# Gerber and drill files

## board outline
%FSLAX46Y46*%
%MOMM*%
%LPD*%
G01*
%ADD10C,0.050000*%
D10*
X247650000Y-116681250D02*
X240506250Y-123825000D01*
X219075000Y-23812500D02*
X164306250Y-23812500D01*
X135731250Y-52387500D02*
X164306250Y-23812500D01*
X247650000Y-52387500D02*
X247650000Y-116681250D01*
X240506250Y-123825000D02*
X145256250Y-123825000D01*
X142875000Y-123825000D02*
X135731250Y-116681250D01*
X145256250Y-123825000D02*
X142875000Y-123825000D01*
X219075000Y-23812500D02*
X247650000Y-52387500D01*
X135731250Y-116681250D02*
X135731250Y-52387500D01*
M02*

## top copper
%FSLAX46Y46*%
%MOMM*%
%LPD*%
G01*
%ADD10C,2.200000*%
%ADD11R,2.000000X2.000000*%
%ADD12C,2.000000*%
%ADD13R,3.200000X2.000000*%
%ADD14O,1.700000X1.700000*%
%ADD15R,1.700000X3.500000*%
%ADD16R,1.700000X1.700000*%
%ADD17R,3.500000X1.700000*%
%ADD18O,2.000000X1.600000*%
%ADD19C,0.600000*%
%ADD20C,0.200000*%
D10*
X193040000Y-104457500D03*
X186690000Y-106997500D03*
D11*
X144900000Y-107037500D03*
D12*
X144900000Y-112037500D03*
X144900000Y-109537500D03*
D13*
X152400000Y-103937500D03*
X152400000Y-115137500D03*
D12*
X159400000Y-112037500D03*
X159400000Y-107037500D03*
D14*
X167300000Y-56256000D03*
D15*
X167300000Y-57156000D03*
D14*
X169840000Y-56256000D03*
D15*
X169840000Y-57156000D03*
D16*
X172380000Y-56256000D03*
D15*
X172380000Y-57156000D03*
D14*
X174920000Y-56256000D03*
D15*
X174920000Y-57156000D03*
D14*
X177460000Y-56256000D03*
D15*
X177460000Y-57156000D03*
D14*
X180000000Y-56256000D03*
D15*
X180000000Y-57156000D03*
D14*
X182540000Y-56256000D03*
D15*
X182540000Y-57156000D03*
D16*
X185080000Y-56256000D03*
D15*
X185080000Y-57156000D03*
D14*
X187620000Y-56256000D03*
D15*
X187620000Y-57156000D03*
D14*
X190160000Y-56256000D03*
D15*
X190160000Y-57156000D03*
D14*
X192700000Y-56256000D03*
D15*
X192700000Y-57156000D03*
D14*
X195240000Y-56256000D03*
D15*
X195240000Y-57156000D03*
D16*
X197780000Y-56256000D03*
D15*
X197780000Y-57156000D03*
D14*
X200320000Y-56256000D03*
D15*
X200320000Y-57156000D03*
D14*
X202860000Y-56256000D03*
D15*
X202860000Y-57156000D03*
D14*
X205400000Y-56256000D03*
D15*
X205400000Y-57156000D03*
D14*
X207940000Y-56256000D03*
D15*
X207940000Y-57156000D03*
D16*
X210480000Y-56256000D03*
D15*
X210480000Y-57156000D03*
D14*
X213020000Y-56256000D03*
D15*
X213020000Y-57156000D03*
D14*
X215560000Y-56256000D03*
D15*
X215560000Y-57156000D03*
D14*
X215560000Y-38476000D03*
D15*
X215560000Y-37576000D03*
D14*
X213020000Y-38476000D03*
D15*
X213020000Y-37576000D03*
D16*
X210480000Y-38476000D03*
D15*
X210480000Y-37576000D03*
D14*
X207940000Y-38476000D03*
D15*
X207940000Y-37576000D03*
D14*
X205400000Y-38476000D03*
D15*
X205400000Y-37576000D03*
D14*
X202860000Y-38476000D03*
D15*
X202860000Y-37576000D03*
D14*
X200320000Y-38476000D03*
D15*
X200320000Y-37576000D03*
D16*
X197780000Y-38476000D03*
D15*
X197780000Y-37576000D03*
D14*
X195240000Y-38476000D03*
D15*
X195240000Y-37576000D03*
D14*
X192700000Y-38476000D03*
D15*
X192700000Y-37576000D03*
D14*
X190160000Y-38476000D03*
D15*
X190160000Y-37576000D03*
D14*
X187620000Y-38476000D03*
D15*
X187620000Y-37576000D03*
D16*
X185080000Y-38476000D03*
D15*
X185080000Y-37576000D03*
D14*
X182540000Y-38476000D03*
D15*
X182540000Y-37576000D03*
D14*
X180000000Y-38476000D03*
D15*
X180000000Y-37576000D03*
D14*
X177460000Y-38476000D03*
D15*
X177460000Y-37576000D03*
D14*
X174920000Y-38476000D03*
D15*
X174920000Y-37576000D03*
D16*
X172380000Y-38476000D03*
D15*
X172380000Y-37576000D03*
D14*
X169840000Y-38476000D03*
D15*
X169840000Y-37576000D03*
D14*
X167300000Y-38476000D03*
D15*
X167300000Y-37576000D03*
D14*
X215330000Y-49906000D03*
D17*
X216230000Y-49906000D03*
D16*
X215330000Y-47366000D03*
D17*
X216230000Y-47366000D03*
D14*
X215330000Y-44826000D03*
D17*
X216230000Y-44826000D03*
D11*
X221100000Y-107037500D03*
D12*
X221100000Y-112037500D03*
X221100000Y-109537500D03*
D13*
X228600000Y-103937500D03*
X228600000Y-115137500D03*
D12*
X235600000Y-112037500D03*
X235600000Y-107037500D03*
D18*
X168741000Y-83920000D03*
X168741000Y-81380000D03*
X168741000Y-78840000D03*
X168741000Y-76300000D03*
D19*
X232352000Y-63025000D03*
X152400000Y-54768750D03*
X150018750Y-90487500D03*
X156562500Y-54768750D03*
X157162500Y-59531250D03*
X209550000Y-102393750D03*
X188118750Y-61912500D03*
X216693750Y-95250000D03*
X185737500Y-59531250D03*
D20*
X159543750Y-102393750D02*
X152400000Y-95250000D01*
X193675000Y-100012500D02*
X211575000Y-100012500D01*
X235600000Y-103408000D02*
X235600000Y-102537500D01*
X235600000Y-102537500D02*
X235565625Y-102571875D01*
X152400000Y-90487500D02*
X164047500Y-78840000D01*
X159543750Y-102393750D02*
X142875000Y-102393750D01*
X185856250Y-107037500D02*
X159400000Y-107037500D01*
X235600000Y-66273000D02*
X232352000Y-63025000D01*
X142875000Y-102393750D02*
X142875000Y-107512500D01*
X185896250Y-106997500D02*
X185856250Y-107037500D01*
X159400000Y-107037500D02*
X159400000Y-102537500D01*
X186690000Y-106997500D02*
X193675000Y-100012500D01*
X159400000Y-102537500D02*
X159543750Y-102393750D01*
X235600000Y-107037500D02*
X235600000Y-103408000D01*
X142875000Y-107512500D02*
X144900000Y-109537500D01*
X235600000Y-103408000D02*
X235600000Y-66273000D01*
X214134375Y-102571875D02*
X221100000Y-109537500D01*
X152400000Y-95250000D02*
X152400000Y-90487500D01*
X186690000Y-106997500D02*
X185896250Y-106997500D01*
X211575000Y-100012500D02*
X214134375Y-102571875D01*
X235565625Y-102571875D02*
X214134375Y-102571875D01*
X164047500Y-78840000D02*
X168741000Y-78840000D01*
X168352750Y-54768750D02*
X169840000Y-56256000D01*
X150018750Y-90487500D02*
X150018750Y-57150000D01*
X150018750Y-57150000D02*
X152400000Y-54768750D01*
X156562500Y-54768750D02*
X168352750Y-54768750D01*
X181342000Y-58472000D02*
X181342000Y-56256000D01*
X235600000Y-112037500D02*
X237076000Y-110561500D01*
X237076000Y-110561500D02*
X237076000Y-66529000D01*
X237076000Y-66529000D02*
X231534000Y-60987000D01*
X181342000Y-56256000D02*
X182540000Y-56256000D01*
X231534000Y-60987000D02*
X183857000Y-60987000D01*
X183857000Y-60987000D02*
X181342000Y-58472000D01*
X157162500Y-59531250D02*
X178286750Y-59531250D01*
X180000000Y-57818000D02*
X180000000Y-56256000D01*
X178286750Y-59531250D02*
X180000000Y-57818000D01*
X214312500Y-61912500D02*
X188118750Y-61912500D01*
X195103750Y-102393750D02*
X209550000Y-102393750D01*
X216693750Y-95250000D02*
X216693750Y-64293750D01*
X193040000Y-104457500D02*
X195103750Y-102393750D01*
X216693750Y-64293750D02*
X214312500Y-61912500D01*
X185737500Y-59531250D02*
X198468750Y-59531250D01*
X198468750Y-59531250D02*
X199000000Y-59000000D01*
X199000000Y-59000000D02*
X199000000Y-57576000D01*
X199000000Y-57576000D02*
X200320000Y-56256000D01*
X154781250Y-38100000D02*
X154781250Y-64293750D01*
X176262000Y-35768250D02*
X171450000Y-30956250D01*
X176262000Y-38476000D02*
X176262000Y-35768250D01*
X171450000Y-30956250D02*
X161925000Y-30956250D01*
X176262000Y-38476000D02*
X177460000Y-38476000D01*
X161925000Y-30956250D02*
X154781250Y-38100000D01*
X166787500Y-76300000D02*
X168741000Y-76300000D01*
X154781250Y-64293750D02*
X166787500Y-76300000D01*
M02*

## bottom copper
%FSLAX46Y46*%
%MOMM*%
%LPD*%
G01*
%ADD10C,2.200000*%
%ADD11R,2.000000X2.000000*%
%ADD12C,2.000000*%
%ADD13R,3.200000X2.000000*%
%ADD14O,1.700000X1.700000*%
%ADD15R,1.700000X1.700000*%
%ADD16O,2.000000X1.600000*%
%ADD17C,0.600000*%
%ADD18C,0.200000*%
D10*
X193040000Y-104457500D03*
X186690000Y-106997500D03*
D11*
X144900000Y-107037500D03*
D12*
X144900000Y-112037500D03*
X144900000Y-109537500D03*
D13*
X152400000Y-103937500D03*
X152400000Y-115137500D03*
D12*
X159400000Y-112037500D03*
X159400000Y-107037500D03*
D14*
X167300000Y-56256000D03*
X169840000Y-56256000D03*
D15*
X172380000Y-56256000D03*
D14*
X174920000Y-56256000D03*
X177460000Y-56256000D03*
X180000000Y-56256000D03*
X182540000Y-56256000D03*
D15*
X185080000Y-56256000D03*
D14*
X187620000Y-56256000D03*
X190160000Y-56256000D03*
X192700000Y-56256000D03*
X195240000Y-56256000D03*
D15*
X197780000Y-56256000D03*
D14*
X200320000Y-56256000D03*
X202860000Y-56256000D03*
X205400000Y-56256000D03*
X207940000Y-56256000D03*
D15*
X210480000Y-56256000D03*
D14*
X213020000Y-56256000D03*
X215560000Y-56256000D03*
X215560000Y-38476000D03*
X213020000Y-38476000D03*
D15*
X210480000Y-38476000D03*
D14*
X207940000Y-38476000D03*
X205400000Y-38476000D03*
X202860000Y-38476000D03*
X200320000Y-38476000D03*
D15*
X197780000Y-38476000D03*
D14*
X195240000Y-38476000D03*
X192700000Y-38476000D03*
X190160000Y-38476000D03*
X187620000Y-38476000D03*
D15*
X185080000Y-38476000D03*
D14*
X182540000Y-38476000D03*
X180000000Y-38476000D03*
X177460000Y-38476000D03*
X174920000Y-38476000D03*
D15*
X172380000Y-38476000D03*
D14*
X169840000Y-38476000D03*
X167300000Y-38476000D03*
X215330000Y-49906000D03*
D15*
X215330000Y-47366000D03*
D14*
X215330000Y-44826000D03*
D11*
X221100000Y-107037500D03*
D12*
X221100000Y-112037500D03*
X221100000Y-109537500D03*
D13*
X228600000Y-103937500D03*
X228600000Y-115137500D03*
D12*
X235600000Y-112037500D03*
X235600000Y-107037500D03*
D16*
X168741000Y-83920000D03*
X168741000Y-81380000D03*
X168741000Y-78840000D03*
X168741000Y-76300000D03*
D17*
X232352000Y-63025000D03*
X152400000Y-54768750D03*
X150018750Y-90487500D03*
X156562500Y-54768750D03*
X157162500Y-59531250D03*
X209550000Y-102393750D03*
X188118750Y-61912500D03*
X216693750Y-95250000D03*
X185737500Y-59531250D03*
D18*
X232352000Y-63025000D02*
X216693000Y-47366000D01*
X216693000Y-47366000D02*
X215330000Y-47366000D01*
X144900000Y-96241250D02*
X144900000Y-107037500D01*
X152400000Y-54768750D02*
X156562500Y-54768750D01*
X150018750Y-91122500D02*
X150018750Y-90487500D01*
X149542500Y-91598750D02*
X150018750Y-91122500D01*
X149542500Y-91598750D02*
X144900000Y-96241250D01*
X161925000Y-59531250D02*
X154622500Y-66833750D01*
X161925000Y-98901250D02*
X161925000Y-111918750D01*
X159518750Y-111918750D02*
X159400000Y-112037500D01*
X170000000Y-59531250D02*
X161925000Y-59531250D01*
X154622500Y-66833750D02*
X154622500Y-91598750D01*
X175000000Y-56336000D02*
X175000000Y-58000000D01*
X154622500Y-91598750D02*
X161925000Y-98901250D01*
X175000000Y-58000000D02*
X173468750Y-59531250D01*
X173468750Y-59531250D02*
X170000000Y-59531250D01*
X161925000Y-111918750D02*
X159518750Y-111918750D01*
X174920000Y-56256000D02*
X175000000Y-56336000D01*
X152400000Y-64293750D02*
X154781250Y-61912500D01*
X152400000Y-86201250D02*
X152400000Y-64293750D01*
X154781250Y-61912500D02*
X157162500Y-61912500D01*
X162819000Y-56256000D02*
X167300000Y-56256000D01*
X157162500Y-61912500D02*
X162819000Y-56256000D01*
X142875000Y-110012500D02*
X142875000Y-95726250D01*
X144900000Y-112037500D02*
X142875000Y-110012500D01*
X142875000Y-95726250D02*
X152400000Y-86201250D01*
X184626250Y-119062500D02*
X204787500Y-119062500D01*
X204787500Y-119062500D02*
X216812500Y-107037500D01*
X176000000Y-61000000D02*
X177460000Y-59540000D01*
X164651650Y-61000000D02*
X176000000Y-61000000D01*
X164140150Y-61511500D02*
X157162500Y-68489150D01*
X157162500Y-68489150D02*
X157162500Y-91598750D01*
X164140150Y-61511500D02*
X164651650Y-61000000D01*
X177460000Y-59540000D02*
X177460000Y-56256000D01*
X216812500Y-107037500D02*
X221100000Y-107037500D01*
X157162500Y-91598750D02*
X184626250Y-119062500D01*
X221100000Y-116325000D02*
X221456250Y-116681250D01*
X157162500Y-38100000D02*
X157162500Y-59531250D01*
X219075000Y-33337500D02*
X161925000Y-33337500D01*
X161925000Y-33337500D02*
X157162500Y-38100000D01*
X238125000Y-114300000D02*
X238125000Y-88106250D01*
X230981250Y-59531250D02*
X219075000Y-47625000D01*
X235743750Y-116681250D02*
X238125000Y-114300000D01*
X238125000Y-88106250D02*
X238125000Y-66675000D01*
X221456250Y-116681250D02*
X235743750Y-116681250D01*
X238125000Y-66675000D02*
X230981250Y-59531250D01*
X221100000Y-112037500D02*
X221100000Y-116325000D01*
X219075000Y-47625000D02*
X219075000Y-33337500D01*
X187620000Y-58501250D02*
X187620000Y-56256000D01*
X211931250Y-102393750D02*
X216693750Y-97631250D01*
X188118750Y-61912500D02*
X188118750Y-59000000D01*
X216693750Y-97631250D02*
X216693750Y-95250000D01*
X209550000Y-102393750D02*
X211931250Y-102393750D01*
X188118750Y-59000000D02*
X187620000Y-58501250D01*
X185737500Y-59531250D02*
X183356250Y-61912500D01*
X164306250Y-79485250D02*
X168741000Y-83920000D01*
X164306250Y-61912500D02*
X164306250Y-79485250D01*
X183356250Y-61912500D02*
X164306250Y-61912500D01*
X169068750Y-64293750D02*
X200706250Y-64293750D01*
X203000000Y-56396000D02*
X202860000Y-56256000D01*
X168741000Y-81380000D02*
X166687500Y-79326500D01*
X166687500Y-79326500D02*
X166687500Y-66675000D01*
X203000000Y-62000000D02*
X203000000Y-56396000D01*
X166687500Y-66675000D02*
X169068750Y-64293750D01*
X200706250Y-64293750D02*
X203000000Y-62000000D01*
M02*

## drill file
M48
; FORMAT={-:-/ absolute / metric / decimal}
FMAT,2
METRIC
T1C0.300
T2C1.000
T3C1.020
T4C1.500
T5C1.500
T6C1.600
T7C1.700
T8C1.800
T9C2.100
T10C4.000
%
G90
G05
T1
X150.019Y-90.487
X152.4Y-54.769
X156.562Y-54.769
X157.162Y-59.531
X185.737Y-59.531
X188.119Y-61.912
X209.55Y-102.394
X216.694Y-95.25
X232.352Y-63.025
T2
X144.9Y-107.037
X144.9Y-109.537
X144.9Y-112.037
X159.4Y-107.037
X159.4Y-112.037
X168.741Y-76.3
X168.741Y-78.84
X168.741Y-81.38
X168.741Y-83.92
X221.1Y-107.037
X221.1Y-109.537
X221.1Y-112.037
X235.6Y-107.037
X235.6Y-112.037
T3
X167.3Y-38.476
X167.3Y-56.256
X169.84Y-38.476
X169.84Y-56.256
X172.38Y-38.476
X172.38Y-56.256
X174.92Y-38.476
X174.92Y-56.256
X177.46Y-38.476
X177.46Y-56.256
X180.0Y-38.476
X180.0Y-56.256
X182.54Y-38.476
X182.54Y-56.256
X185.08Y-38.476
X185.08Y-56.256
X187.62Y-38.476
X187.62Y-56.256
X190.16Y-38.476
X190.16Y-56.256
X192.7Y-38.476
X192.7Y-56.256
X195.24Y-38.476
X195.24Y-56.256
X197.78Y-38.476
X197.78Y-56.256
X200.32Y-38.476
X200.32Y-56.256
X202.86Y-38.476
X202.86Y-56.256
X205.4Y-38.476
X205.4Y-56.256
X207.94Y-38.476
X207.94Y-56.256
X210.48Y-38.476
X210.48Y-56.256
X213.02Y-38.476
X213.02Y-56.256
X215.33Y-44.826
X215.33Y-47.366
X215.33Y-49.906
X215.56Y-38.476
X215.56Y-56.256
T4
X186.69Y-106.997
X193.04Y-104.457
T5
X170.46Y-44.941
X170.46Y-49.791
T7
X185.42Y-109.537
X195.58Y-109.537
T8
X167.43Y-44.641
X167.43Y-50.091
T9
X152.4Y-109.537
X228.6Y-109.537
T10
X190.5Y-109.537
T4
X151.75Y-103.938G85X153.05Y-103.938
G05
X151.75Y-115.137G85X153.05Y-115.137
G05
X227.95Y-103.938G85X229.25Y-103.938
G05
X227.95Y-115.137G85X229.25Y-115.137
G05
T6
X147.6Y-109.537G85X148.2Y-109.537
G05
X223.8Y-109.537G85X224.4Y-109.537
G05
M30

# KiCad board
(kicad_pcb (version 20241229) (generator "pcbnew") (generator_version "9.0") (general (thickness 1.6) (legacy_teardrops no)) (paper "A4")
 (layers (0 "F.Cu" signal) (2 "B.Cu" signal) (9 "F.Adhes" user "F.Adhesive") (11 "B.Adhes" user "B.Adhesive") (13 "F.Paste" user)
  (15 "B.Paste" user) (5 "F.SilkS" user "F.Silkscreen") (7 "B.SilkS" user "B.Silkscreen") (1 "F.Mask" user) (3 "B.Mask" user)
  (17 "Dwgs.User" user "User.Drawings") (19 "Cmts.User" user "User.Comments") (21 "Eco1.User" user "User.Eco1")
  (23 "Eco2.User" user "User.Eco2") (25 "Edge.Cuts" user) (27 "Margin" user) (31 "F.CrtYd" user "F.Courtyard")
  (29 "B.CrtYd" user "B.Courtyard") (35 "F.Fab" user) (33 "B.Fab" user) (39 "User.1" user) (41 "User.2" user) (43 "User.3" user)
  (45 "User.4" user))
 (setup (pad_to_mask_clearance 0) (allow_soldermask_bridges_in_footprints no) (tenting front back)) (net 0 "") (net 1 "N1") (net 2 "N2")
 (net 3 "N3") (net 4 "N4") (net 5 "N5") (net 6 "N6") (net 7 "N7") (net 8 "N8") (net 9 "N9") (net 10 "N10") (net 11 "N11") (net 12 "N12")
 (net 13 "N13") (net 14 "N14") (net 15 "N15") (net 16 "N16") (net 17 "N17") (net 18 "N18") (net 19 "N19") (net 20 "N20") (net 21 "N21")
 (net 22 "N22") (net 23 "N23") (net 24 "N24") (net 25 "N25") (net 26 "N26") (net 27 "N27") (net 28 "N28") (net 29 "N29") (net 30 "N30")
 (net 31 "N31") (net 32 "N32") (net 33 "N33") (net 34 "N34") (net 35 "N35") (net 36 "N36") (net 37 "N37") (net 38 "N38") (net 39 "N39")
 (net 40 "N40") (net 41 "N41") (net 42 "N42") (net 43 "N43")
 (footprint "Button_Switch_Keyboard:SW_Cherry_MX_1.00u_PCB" (layer "F.Cu") (at 193.04 104.4575)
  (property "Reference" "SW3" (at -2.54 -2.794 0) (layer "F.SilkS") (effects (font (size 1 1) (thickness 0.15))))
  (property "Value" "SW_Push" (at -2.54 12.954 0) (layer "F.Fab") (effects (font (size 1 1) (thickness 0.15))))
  (pad "" np_thru_hole circle (at -7.62 5.08) (size 1.7 1.7) (drill 1.7) (layers "*.Cu" "*.Mask"))
  (pad "" np_thru_hole circle (at -2.54 5.08) (size 4 4) (drill 4) (layers "*.Cu" "*.Mask"))
  (pad "" np_thru_hole circle (at 2.54 5.08) (size 1.7 1.7) (drill 1.7) (layers "*.Cu" "*.Mask"))
  (pad "1" thru_hole circle (at 0 0) (size 2.2 2.2) (drill 1.5) (layers "*.Cu" "*.Mask") (remove_unused_layers no) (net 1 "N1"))
  (pad "2" thru_hole circle (at -6.35 2.54) (size 2.2 2.2) (drill 1.5) (layers "*.Cu" "*.Mask") (remove_unused_layers no) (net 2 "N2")))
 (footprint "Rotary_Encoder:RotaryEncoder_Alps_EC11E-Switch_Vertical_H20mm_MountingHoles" (layer "F.Cu") (at 144.9 107.0375)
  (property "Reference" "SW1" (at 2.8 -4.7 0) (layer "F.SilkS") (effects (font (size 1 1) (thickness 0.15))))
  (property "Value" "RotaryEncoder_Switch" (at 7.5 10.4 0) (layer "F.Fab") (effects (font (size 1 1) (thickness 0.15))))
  (pad "" np_thru_hole oval (at 3 2.5) (size 2.2 1.6) (drill oval 2.2 1.6) (layers "*.Mask"))
  (pad "" np_thru_hole circle (at 7.5 2.5) (size 2.1 2.1) (drill 2.1) (layers "*.Mask"))
  (pad "A" thru_hole rect (at 0 0) (size 2 2) (drill 1) (layers "*.Cu" "*.Mask") (remove_unused_layers no) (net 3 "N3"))
  (pad "B" thru_hole circle (at 0 5) (size 2 2) (drill 1) (layers "*.Cu" "*.Mask") (remove_unused_layers no) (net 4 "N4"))
  (pad "C" thru_hole circle (at 0 2.5) (size 2 2) (drill 1) (layers "*.Cu" "*.Mask") (remove_unused_layers no) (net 2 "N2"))
  (pad "MP" thru_hole rect (at 7.5 -3.1) (size 3.2 2) (drill oval 2.8 1.5) (layers "*.Cu" "*.Mask") (remove_unused_layers no))
  (pad "MP" thru_hole rect (at 7.5 8.1) (size 3.2 2) (drill oval 2.8 1.5) (layers "*.Cu" "*.Mask") (remove_unused_layers no))
  (pad "S1" thru_hole circle (at 14.5 5) (size 2 2) (drill 1) (layers "*.Cu" "*.Mask") (remove_unused_layers no) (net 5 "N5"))
  (pad "S2" thru_hole circle (at 14.5 0) (size 2 2) (drill 1) (layers "*.Cu" "*.Mask") (remove_unused_layers no) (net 2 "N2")))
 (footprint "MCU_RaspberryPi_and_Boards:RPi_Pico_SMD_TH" (layer "F.Cu") (at 191.43 47.366 90)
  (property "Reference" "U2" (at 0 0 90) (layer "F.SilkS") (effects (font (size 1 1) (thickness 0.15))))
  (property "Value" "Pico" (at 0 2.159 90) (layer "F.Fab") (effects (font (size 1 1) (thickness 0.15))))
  (pad "" np_thru_hole oval (at -2.725 -24 90) (size 1.8 1.8) (drill 1.8) (layers "*.Cu" "*.Mask"))
  (pad "" np_thru_hole oval (at -2.425 -20.97 90) (size 1.5 1.5) (drill 1.5) (layers "*.Cu" "*.Mask"))
  (pad "" np_thru_hole oval (at 2.425 -20.97 90) (size 1.5 1.5) (drill 1.5) (layers "*.Cu" "*.Mask"))
  (pad "" np_thru_hole oval (at 2.725 -24 90) (size 1.8 1.8) (drill 1.8) (layers "*.Cu" "*.Mask"))
  (pad "1" thru_hole oval (at -8.89 -24.13 90) (size 1.7 1.7) (drill 1.02) (layers "*.Cu" "*.Mask") (remove_unused_layers no) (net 4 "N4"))
  (pad "1" smd rect (at -8.89 -24.13 90) (size 3.5 1.7) (drill (offset -0.9 0)) (layers "F.Cu" "F.Mask") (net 4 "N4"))
  (pad "2" thru_hole oval (at -8.89 -21.59 90) (size 1.7 1.7) (drill 1.02) (layers "*.Cu" "*.Mask") (remove_unused_layers no) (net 3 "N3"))
  (pad "2" smd rect (at -8.89 -21.59 90) (size 3.5 1.7) (drill (offset -0.9 0)) (layers "F.Cu" "F.Mask") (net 3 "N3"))
  (pad "3" thru_hole rect (at -8.89 -19.05 90) (size 1.7 1.7) (drill 1.02) (layers "*.Cu" "*.Mask") (remove_unused_layers no) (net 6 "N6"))
  (pad "3" smd rect (at -8.89 -19.05 90) (size 3.5 1.7) (drill (offset -0.9 0)) (layers "F.Cu" "F.Mask") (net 6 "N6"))
  (pad "4" thru_hole oval (at -8.89 -16.51 90) (size 1.7 1.7) (drill 1.02) (layers "*.Cu" "*.Mask") (remove_unused_layers no) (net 5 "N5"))
  (pad "4" smd rect (at -8.89 -16.51 90) (size 3.5 1.7) (drill (offset -0.9 0)) (layers "F.Cu" "F.Mask") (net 5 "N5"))
  (pad "5" thru_hole oval (at -8.89 -13.97 90) (size 1.7 1.7) (drill 1.02) (layers "*.Cu" "*.Mask") (remove_unused_layers no) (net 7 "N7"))
  (pad "5" smd rect (at -8.89 -13.97 90) (size 3.5 1.7) (drill (offset -0.9 0)) (layers "F.Cu" "F.Mask") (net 7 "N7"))
  (pad "6" thru_hole oval (at -8.89 -11.43 90) (size 1.7 1.7) (drill 1.02) (layers "*.Cu" "*.Mask") (remove_unused_layers no) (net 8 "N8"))
  (pad "6" smd rect (at -8.89 -11.43 90) (size 3.5 1.7) (drill (offset -0.9 0)) (layers "F.Cu" "F.Mask") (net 8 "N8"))
  (pad "7" thru_hole oval (at -8.89 -8.89 90) (size 1.7 1.7) (drill 1.02) (layers "*.Cu" "*.Mask") (remove_unused_layers no) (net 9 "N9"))
  (pad "7" smd rect (at -8.89 -8.89 90) (size 3.5 1.7) (drill (offset -0.9 0)) (layers "F.Cu" "F.Mask") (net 9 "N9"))
  (pad "8" thru_hole rect (at -8.89 -6.35 90) (size 1.7 1.7) (drill 1.02) (layers "*.Cu" "*.Mask") (remove_unused_layers no) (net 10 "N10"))
  (pad "8" smd rect (at -8.89 -6.35 90) (size 3.5 1.7) (drill (offset -0.9 0)) (layers "F.Cu" "F.Mask") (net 10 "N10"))
  (pad "9" thru_hole oval (at -8.89 -3.81 90) (size 1.7 1.7) (drill 1.02) (layers "*.Cu" "*.Mask") (remove_unused_layers no) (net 1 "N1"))
  (pad "9" smd rect (at -8.89 -3.81 90) (size 3.5 1.7) (drill (offset -0.9 0)) (layers "F.Cu" "F.Mask") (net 1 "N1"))
  (pad "10" thru_hole oval (at -8.89 -1.27 90) (size 1.7 1.7) (drill 1.02) (layers "*.Cu" "*.Mask") (remove_unused_layers no) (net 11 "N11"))
  (pad "10" smd rect (at -8.89 -1.27 90) (size 3.5 1.7) (drill (offset -0.9 0)) (layers "F.Cu" "F.Mask") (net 11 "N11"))
  (pad "11" thru_hole oval (at -8.89 1.27 90) (size 1.7 1.7) (drill 1.02) (layers "*.Cu" "*.Mask") (remove_unused_layers no) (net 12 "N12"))
  (pad "11" smd rect (at -8.89 1.27 90) (size 3.5 1.7) (drill (offset -0.9 0)) (layers "F.Cu" "F.Mask") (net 12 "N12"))
  (pad "12" thru_hole oval (at -8.89 3.81 90) (size 1.7 1.7) (drill 1.02) (layers "*.Cu" "*.Mask") (remove_unused_layers no) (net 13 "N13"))
  (pad "12" smd rect (at -8.89 3.81 90) (size 3.5 1.7) (drill (offset -0.9 0)) (layers "F.Cu" "F.Mask") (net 13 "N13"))
  (pad "13" thru_hole rect (at -8.89 6.35 90) (size 1.7 1.7) (drill 1.02) (layers "*.Cu" "*.Mask") (remove_unused_layers no) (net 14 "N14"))
  (pad "13" smd rect (at -8.89 6.35 90) (size 3.5 1.7) (drill (offset -0.9 0)) (layers "F.Cu" "F.Mask") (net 14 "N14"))
  (pad "14" thru_hole oval (at -8.89 8.89 90) (size 1.7 1.7) (drill 1.02) (layers "*.Cu" "*.Mask") (remove_unused_layers no) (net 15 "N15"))
  (pad "14" smd rect (at -8.89 8.89 90) (size 3.5 1.7) (drill (offset -0.9 0)) (layers "F.Cu" "F.Mask") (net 15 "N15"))
  (pad "15" thru_hole oval (at -8.89 11.43 90) (size 1.7 1.7) (drill 1.02) (layers "*.Cu" "*.Mask") (remove_unused_layers no) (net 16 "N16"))
  (pad "15" smd rect (at -8.89 11.43 90) (size 3.5 1.7) (drill (offset -0.9 0)) (layers "F.Cu" "F.Mask") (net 16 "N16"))
  (pad "16" thru_hole oval (at -8.89 13.97 90) (size 1.7 1.7) (drill 1.02) (layers "*.Cu" "*.Mask") (remove_unused_layers no) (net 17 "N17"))
  (pad "16" smd rect (at -8.89 13.97 90) (size 3.5 1.7) (drill (offset -0.9 0)) (layers "F.Cu" "F.Mask") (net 17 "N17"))
  (pad "17" thru_hole oval (at -8.89 16.51 90) (size 1.7 1.7) (drill 1.02) (layers "*.Cu" "*.Mask") (remove_unused_layers no) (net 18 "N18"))
  (pad "17" smd rect (at -8.89 16.51 90) (size 3.5 1.7) (drill (offset -0.9 0)) (layers "F.Cu" "F.Mask") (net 18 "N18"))
  (pad "18" thru_hole rect (at -8.89 19.05 90) (size 1.7 1.7) (drill 1.02) (layers "*.Cu" "*.Mask") (remove_unused_layers no) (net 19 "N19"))
  (pad "18" smd rect (at -8.89 19.05 90) (size 3.5 1.7) (drill (offset -0.9 0)) (layers "F.Cu" "F.Mask") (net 19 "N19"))
  (pad "19" thru_hole oval (at -8.89 21.59 90) (size 1.7 1.7) (drill 1.02) (layers "*.Cu" "*.Mask") (remove_unused_layers no) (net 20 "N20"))
  (pad "19" smd rect (at -8.89 21.59 90) (size 3.5 1.7) (drill (offset -0.9 0)) (layers "F.Cu" "F.Mask") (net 20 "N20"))
  (pad "20" thru_hole oval (at -8.89 24.13 90) (size 1.7 1.7) (drill 1.02) (layers "*.Cu" "*.Mask") (remove_unused_layers no) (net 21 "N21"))
  (pad "20" smd rect (at -8.89 24.13 90) (size 3.5 1.7) (drill (offset -0.9 0)) (layers "F.Cu" "F.Mask") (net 21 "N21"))
  (pad "21" thru_hole oval (at 8.89 24.13 90) (size 1.7 1.7) (drill 1.02) (layers "*.Cu" "*.Mask") (remove_unused_layers no) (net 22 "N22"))
  (pad "21" smd rect (at 8.89 24.13 90) (size 3.5 1.7) (drill (offset 0.9 0)) (layers "F.Cu" "F.Mask") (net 22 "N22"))
  (pad "22" thru_hole oval (at 8.89 21.59 90) (size 1.7 1.7) (drill 1.02) (layers "*.Cu" "*.Mask") (remove_unused_layers no) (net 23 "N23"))
  (pad "22" smd rect (at 8.89 21.59 90) (size 3.5 1.7) (drill (offset 0.9 0)) (layers "F.Cu" "F.Mask") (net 23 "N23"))
  (pad "23" thru_hole rect (at 8.89 19.05 90) (size 1.7 1.7) (drill 1.02) (layers "*.Cu" "*.Mask") (remove_unused_layers no) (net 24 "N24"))
  (pad "23" smd rect (at 8.89 19.05 90) (size 3.5 1.7) (drill (offset 0.9 0)) (layers "F.Cu" "F.Mask") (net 24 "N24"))
  (pad "24" thru_hole oval (at 8.89 16.51 90) (size 1.7 1.7) (drill 1.02) (layers "*.Cu" "*.Mask") (remove_unused_layers no) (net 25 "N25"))
  (pad "24" smd rect (at 8.89 16.51 90) (size 3.5 1.7) (drill (offset 0.9 0)) (layers "F.Cu" "F.Mask") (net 25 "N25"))
  (pad "25" thru_hole oval (at 8.89 13.97 90) (size 1.7 1.7) (drill 1.02) (layers "*.Cu" "*.Mask") (remove_unused_layers no) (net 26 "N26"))
  (pad "25" smd rect (at 8.89 13.97 90) (size 3.5 1.7) (drill (offset 0.9 0)) (layers "F.Cu" "F.Mask") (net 26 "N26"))
  (pad "26" thru_hole oval (at 8.89 11.43 90) (size 1.7 1.7) (drill 1.02) (layers "*.Cu" "*.Mask") (remove_unused_layers no) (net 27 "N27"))
  (pad "26" smd rect (at 8.89 11.43 90) (size 3.5 1.7) (drill (offset 0.9 0)) (layers "F.Cu" "F.Mask") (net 27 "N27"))
  (pad "27" thru_hole oval (at 8.89 8.89 90) (size 1.7 1.7) (drill 1.02) (layers "*.Cu" "*.Mask") (remove_unused_layers no) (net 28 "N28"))
  (pad "27" smd rect (at 8.89 8.89 90) (size 3.5 1.7) (drill (offset 0.9 0)) (layers "F.Cu" "F.Mask") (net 28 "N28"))
  (pad "28" thru_hole rect (at 8.89 6.35 90) (size 1.7 1.7) (drill 1.02) (layers "*.Cu" "*.Mask") (remove_unused_layers no) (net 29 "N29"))
  (pad "28" smd rect (at 8.89 6.35 90) (size 3.5 1.7) (drill (offset 0.9 0)) (layers "F.Cu" "F.Mask") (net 29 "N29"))
  (pad "29" thru_hole oval (at 8.89 3.81 90) (size 1.7 1.7) (drill 1.02) (layers "*.Cu" "*.Mask") (remove_unused_layers no) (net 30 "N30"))
  (pad "29" smd rect (at 8.89 3.81 90) (size 3.5 1.7) (drill (offset 0.9 0)) (layers "F.Cu" "F.Mask") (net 30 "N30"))
  (pad "30" thru_hole oval (at 8.89 1.27 90) (size 1.7 1.7) (drill 1.02) (layers "*.Cu" "*.Mask") (remove_unused_layers no) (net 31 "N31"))
  (pad "30" smd rect (at 8.89 1.27 90) (size 3.5 1.7) (drill (offset 0.9 0)) (layers "F.Cu" "F.Mask") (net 31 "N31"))
  (pad "31" thru_hole oval (at 8.89 -1.27 90) (size 1.7 1.7) (drill 1.02) (layers "*.Cu" "*.Mask") (remove_unused_layers no) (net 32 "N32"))
  (pad "31" smd rect (at 8.89 -1.27 90) (size 3.5 1.7) (drill (offset 0.9 0)) (layers "F.Cu" "F.Mask") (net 32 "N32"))
  (pad "32" thru_hole oval (at 8.89 -3.81 90) (size 1.7 1.7) (drill 1.02) (layers "*.Cu" "*.Mask") (remove_unused_layers no) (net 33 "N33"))
  (pad "32" smd rect (at 8.89 -3.81 90) (size 3.5 1.7) (drill (offset 0.9 0)) (layers "F.Cu" "F.Mask") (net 33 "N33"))
  (pad "33" thru_hole rect (at 8.89 -6.35 90) (size 1.7 1.7) (drill 1.02) (layers "*.Cu" "*.Mask") (remove_unused_layers no) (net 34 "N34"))
  (pad "33" smd rect (at 8.89 -6.35 90) (size 3.5 1.7) (drill (offset 0.9 0)) (layers "F.Cu" "F.Mask") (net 34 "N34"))
  (pad "34" thru_hole oval (at 8.89 -8.89 90) (size 1.7 1.7) (drill 1.02) (layers "*.Cu" "*.Mask") (remove_unused_layers no) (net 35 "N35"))
  (pad "34" smd rect (at 8.89 -8.89 90) (size 3.5 1.7) (drill (offset 0.9 0)) (layers "F.Cu" "F.Mask") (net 35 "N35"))
  (pad "35" thru_hole oval (at 8.89 -11.43 90) (size 1.7 1.7) (drill 1.02) (layers "*.Cu" "*.Mask") (remove_unused_layers no) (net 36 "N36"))
  (pad "35" smd rect (at 8.89 -11.43 90) (size 3.5 1.7) (drill (offset 0.9 0)) (layers "F.Cu" "F.Mask") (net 36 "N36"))
  (pad "36" thru_hole oval (at 8.89 -13.97 90) (size 1.7 1.7) (drill 1.02) (layers "*.Cu" "*.Mask") (remove_unused_layers no) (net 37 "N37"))
  (pad "36" smd rect (at 8.89 -13.97 90) (size 3.5 1.7) (drill (offset 0.9 0)) (layers "F.Cu" "F.Mask") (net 37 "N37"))
  (pad "37" thru_hole oval (at 8.89 -16.51 90) (size 1.7 1.7) (drill 1.02) (layers "*.Cu" "*.Mask") (remove_unused_layers no) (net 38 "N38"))
  (pad "37" smd rect (at 8.89 -16.51 90) (size 3.5 1.7) (drill (offset 0.9 0)) (layers "F.Cu" "F.Mask") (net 38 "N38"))
  (pad "38" thru_hole rect (at 8.89 -19.05 90) (size 1.7 1.7) (drill 1.02) (layers "*.Cu" "*.Mask") (remove_unused_layers no) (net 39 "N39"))
  (pad "38" smd rect (at 8.89 -19.05 90) (size 3.5 1.7) (drill (offset 0.9 0)) (layers "F.Cu" "F.Mask") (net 39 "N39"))
  (pad "39" thru_hole oval (at 8.89 -21.59 90) (size 1.7 1.7) (drill 1.02) (layers "*.Cu" "*.Mask") (remove_unused_layers no) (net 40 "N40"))
  (pad "39" smd rect (at 8.89 -21.59 90) (size 3.5 1.7) (drill (offset 0.9 0)) (layers "F.Cu" "F.Mask") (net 40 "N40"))
  (pad "40" thru_hole oval (at 8.89 -24.13 90) (size 1.7 1.7) (drill 1.02) (layers "*.Cu" "*.Mask") (remove_unused_layers no) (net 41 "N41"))
  (pad "40" smd rect (at 8.89 -24.13 90) (size 3.5 1.7) (drill (offset 0.9 0)) (layers "F.Cu" "F.Mask") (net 41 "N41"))
  (pad "41" thru_hole oval (at -2.54 23.9 90) (size 1.7 1.7) (drill 1.02) (layers "*.Cu" "*.Mask") (remove_unused_layers no) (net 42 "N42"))
  (pad "41" smd rect (at -2.54 23.9 180) (size 3.5 1.7) (drill (offset -0.9 0)) (layers "F.Cu" "F.Mask") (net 42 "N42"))
  (pad "42" thru_hole rect (at 0 23.9 90) (size 1.7 1.7) (drill 1.02) (layers "*.Cu" "*.Mask") (remove_unused_layers no) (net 2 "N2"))
  (pad "42" smd rect (at 0 23.9 180) (size 3.5 1.7) (drill (offset -0.9 0)) (layers "F.Cu" "F.Mask") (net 2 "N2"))
  (pad "43" thru_hole oval (at 2.54 23.9 90) (size 1.7 1.7) (drill 1.02) (layers "*.Cu" "*.Mask") (remove_unused_layers no) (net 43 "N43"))
  (pad "43" smd rect (at 2.54 23.9 180) (size 3.5 1.7) (drill (offset -0.9 0)) (layers "F.Cu" "F.Mask") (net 43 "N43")))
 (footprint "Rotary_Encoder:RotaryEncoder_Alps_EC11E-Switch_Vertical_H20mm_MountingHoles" (layer "F.Cu") (at 221.1 107.0375)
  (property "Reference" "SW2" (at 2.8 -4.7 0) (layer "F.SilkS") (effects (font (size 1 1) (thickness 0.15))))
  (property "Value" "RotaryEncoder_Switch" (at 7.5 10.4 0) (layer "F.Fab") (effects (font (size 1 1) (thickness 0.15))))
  (pad "" np_thru_hole oval (at 3 2.5) (size 2.2 1.6) (drill oval 2.2 1.6) (layers "*.Mask"))
  (pad "" np_thru_hole circle (at 7.5 2.5) (size 2.1 2.1) (drill 2.1) (layers "*.Mask"))
  (pad "A" thru_hole rect (at 0 0) (size 2 2) (drill 1) (layers "*.Cu" "*.Mask") (remove_unused_layers no) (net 7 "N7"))
  (pad "B" thru_hole circle (at 0 5) (size 2 2) (drill 1) (layers "*.Cu" "*.Mask") (remove_unused_layers no) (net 8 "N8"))
  (pad "C" thru_hole circle (at 0 2.5) (size 2 2) (drill 1) (layers "*.Cu" "*.Mask") (remove_unused_layers no) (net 2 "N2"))
  (pad "MP" thru_hole rect (at 7.5 -3.1) (size 3.2 2) (drill oval 2.8 1.5) (layers "*.Cu" "*.Mask") (remove_unused_layers no))
  (pad "MP" thru_hole rect (at 7.5 8.1) (size 3.2 2) (drill oval 2.8 1.5) (layers "*.Cu" "*.Mask") (remove_unused_layers no))
  (pad "S1" thru_hole circle (at 14.5 5) (size 2 2) (drill 1) (layers "*.Cu" "*.Mask") (remove_unused_layers no) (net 9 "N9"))
  (pad "S2" thru_hole circle (at 14.5 0) (size 2 2) (drill 1) (layers "*.Cu" "*.Mask") (remove_unused_layers no) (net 2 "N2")))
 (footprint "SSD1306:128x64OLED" (layer "F.Cu") (at 179.341 80.3 90)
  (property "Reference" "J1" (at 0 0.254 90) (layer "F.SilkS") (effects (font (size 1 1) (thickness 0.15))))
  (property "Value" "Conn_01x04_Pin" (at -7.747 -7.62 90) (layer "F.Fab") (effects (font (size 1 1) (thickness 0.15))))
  (pad "1" thru_hole oval (at -3.62 -10.6 180) (size 2 1.6) (drill 1) (layers "*.Cu" "*.Mask") (remove_unused_layers no) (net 15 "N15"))
  (pad "2" thru_hole oval (at -1.08 -10.6 180) (size 2 1.6) (drill 1) (layers "*.Cu" "*.Mask") (remove_unused_layers no) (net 16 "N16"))
  (pad "3" thru_hole oval (at 1.46 -10.6 180) (size 2 1.6) (drill 1) (layers "*.Cu" "*.Mask") (remove_unused_layers no) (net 2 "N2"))
  (pad "4" thru_hole oval (at 4 -10.6 180) (size 2 1.6) (drill 1) (layers "*.Cu" "*.Mask") (remove_unused_layers no) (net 37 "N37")))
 (gr_line (start 247.65 116.68125) (end 240.50625 123.825) (stroke (width 0.05) (type default)) (layer "Edge.Cuts"))
 (gr_line (start 219.075 23.8125) (end 164.30625 23.8125) (stroke (width 0.05) (type default)) (layer "Edge.Cuts"))
 (gr_line (start 135.73125 52.3875) (end 164.30625 23.8125) (stroke (width 0.05) (type default)) (layer "Edge.Cuts"))
 (gr_line (start 247.65 52.3875) (end 247.65 116.68125) (stroke (width 0.05) (type default)) (layer "Edge.Cuts"))
 (gr_line (start 240.50625 123.825) (end 145.25625 123.825) (stroke (width 0.05) (type default)) (layer "Edge.Cuts"))
 (gr_line (start 142.875 123.825) (end 135.73125 116.68125) (stroke (width 0.05) (type default)) (layer "Edge.Cuts"))
 (gr_line (start 145.25625 123.825) (end 142.875 123.825) (stroke (width 0.05) (type default)) (layer "Edge.Cuts"))
 (gr_line (start 219.075 23.8125) (end 247.65 52.3875) (stroke (width 0.05) (type default)) (layer "Edge.Cuts"))
 (gr_line (start 135.73125 116.68125) (end 135.73125 52.3875) (stroke (width 0.05) (type default)) (layer "Edge.Cuts"))
 (segment (start 159.54375 102.39375) (end 152.4 95.25) (width 0.2) (layer "F.Cu") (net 2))
 (segment (start 193.675 100.0125) (end 211.575 100.0125) (width 0.2) (layer "F.Cu") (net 2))
 (segment (start 235.6 103.408) (end 235.6 102.5375) (width 0.2) (layer "F.Cu") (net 2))
 (segment (start 235.6 102.5375) (end 235.565625 102.571875) (width 0.2) (layer "F.Cu") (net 2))
 (segment (start 152.4 90.4875) (end 164.0475 78.84) (width 0.2) (layer "F.Cu") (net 2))
 (segment (start 159.54375 102.39375) (end 142.875 102.39375) (width 0.2) (layer "F.Cu") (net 2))
 (segment (start 185.85625 107.0375) (end 159.4 107.0375) (width 0.2) (layer "F.Cu") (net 2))
 (segment (start 235.6 66.273) (end 232.352 63.025) (width 0.2) (layer "F.Cu") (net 2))
 (segment (start 142.875 102.39375) (end 142.875 107.5125) (width 0.2) (layer "F.Cu") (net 2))
 (segment (start 185.89625 106.9975) (end 185.85625 107.0375) (width 0.2) (layer "F.Cu") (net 2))
 (segment (start 159.4 107.0375) (end 159.4 102.5375) (width 0.2) (layer "F.Cu") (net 2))
 (segment (start 186.69 106.9975) (end 193.675 100.0125) (width 0.2) (layer "F.Cu") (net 2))
 (segment (start 159.4 102.5375) (end 159.54375 102.39375) (width 0.2) (layer "F.Cu") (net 2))
 (segment (start 235.6 107.0375) (end 235.6 103.408) (width 0.2) (layer "F.Cu") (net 2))
 (segment (start 142.875 107.5125) (end 144.9 109.5375) (width 0.2) (layer "F.Cu") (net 2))
 (segment (start 235.6 103.408) (end 235.6 66.273) (width 0.2) (layer "F.Cu") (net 2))
 (segment (start 214.134375 102.571875) (end 221.1 109.5375) (width 0.2) (layer "F.Cu") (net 2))
 (segment (start 152.4 95.25) (end 152.4 90.4875) (width 0.2) (layer "F.Cu") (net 2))
 (segment (start 186.69 106.9975) (end 185.89625 106.9975) (width 0.2) (layer "F.Cu") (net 2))
 (segment (start 211.575 100.0125) (end 214.134375 102.571875) (width 0.2) (layer "F.Cu") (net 2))
 (segment (start 235.565625 102.571875) (end 214.134375 102.571875) (width 0.2) (layer "F.Cu") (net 2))
 (segment (start 164.0475 78.84) (end 168.741 78.84) (width 0.2) (layer "F.Cu") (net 2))
 (via (at 232.352 63.025) (size 0.6) (drill 0.3) (layers "F.Cu" "B.Cu") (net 2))
 (segment (start 232.352 63.025) (end 216.693 47.366) (width 0.2) (layer "B.Cu") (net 2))
 (segment (start 216.693 47.366) (end 215.33 47.366) (width 0.2) (layer "B.Cu") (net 2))
 (segment (start 168.35275 54.76875) (end 169.84 56.256) (width 0.2) (layer "F.Cu") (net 3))
 (segment (start 150.01875 90.4875) (end 150.01875 57.15) (width 0.2) (layer "F.Cu") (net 3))
 (segment (start 150.01875 57.15) (end 152.4 54.76875) (width 0.2) (layer "F.Cu") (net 3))
 (segment (start 156.5625 54.76875) (end 168.35275 54.76875) (width 0.2) (layer "F.Cu") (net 3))
 (via (at 152.4 54.76875) (size 0.6) (drill 0.3) (layers "F.Cu" "B.Cu") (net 3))
 (via (at 150.01875 90.4875) (size 0.6) (drill 0.3) (layers "F.Cu" "B.Cu") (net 3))
 (via (at 156.5625 54.76875) (size 0.6) (drill 0.3) (layers "F.Cu" "B.Cu") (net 3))
 (segment (start 144.9 96.24125) (end 144.9 107.0375) (width 0.2) (layer "B.Cu") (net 3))
 (segment (start 152.4 54.76875) (end 156.5625 54.76875) (width 0.2) (layer "B.Cu") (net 3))
 (segment (start 150.01875 91.1225) (end 150.01875 90.4875) (width 0.2) (layer "B.Cu") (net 3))
 (segment (start 149.5425 91.59875) (end 150.01875 91.1225) (width 0.2) (layer "B.Cu") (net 3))
 (segment (start 149.5425 91.59875) (end 144.9 96.24125) (width 0.2) (layer "B.Cu") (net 3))
 (segment (start 161.925 59.53125) (end 154.6225 66.83375) (width 0.2) (layer "B.Cu") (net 5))
 (segment (start 161.925 98.90125) (end 161.925 111.91875) (width 0.2) (layer "B.Cu") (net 5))
 (segment (start 159.51875 111.91875) (end 159.4 112.0375) (width 0.2) (layer "B.Cu") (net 5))
 (segment (start 170 59.53125) (end 161.925 59.53125) (width 0.2) (layer "B.Cu") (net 5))
 (segment (start 154.6225 66.83375) (end 154.6225 91.59875) (width 0.2) (layer "B.Cu") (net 5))
 (segment (start 175 56.336) (end 175 58) (width 0.2) (layer "B.Cu") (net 5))
 (segment (start 154.6225 91.59875) (end 161.925 98.90125) (width 0.2) (layer "B.Cu") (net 5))
 (segment (start 175 58) (end 173.46875 59.53125) (width 0.2) (layer "B.Cu") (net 5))
 (segment (start 173.46875 59.53125) (end 170 59.53125) (width 0.2) (layer "B.Cu") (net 5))
 (segment (start 161.925 111.91875) (end 159.51875 111.91875) (width 0.2) (layer "B.Cu") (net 5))
 (segment (start 174.92 56.256) (end 175 56.336) (width 0.2) (layer "B.Cu") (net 5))
 (segment (start 152.4 64.29375) (end 154.78125 61.9125) (width 0.2) (layer "B.Cu") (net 4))
 (segment (start 152.4 86.20125) (end 152.4 64.29375) (width 0.2) (layer "B.Cu") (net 4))
 (segment (start 154.78125 61.9125) (end 157.1625 61.9125) (width 0.2) (layer "B.Cu") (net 4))
 (segment (start 162.819 56.256) (end 167.3 56.256) (width 0.2) (layer "B.Cu") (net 4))
 (segment (start 157.1625 61.9125) (end 162.819 56.256) (width 0.2) (layer "B.Cu") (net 4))
 (segment (start 142.875 110.0125) (end 142.875 95.72625) (width 0.2) (layer "B.Cu") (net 4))
 (segment (start 144.9 112.0375) (end 142.875 110.0125) (width 0.2) (layer "B.Cu") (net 4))
 (segment (start 142.875 95.72625) (end 152.4 86.20125) (width 0.2) (layer "B.Cu") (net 4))
 (segment (start 184.62625 119.0625) (end 204.7875 119.0625) (width 0.2) (layer "B.Cu") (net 7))
 (segment (start 204.7875 119.0625) (end 216.8125 107.0375) (width 0.2) (layer "B.Cu") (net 7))
 (segment (start 176 61) (end 177.46 59.54) (width 0.2) (layer "B.Cu") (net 7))
 (segment (start 164.65165 61) (end 176 61) (width 0.2) (layer "B.Cu") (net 7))
 (segment (start 164.14015 61.5115) (end 157.1625 68.48915) (width 0.2) (layer "B.Cu") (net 7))
 (segment (start 157.1625 68.48915) (end 157.1625 91.59875) (width 0.2) (layer "B.Cu") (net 7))
 (segment (start 164.14015 61.5115) (end 164.65165 61) (width 0.2) (layer "B.Cu") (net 7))
 (segment (start 177.46 59.54) (end 177.46 56.256) (width 0.2) (layer "B.Cu") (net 7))
 (segment (start 216.8125 107.0375) (end 221.1 107.0375) (width 0.2) (layer "B.Cu") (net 7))
 (segment (start 157.1625 91.59875) (end 184.62625 119.0625) (width 0.2) (layer "B.Cu") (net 7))
 (segment (start 181.342 58.472) (end 181.342 56.256) (width 0.2) (layer "F.Cu") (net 9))
 (segment (start 235.6 112.0375) (end 237.076 110.5615) (width 0.2) (layer "F.Cu") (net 9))
 (segment (start 237.076 110.5615) (end 237.076 66.529) (width 0.2) (layer "F.Cu") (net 9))
 (segment (start 237.076 66.529) (end 231.534 60.987) (width 0.2) (layer "F.Cu") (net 9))
 (segment (start 181.342 56.256) (end 182.54 56.256) (width 0.2) (layer "F.Cu") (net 9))
 (segment (start 231.534 60.987) (end 183.857 60.987) (width 0.2) (layer "F.Cu") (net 9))
 (segment (start 183.857 60.987) (end 181.342 58.472) (width 0.2) (layer "F.Cu") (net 9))
 (segment (start 157.1625 59.53125) (end 178.28675 59.53125) (width 0.2) (layer "F.Cu") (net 8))
 (segment (start 180 57.818) (end 180 56.256) (width 0.2) (layer "F.Cu") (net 8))
 (segment (start 178.28675 59.53125) (end 180 57.818) (width 0.2) (layer "F.Cu") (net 8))
 (via (at 157.1625 59.53125) (size 0.6) (drill 0.3) (layers "F.Cu" "B.Cu") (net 8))
 (segment (start 221.1 116.325) (end 221.45625 116.68125) (width 0.2) (layer "B.Cu") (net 8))
 (segment (start 157.1625 38.1) (end 157.1625 59.53125) (width 0.2) (layer "B.Cu") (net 8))
 (segment (start 219.075 33.3375) (end 161.925 33.3375) (width 0.2) (layer "B.Cu") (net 8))
 (segment (start 161.925 33.3375) (end 157.1625 38.1) (width 0.2) (layer "B.Cu") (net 8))
 (segment (start 238.125 114.3) (end 238.125 88.10625) (width 0.2) (layer "B.Cu") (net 8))
 (segment (start 230.98125 59.53125) (end 219.075 47.625) (width 0.2) (layer "B.Cu") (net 8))
 (segment (start 235.74375 116.68125) (end 238.125 114.3) (width 0.2) (layer "B.Cu") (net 8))
 (segment (start 238.125 88.10625) (end 238.125 66.675) (width 0.2) (layer "B.Cu") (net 8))
 (segment (start 221.45625 116.68125) (end 235.74375 116.68125) (width 0.2) (layer "B.Cu") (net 8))
 (segment (start 238.125 66.675) (end 230.98125 59.53125) (width 0.2) (layer "B.Cu") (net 8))
 (segment (start 221.1 112.0375) (end 221.1 116.325) (width 0.2) (layer "B.Cu") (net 8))
 (segment (start 219.075 47.625) (end 219.075 33.3375) (width 0.2) (layer "B.Cu") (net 8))
 (segment (start 214.3125 61.9125) (end 188.11875 61.9125) (width 0.2) (layer "F.Cu") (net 1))
 (segment (start 195.10375 102.39375) (end 209.55 102.39375) (width 0.2) (layer "F.Cu") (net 1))
 (segment (start 216.69375 95.25) (end 216.69375 64.29375) (width 0.2) (layer "F.Cu") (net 1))
 (segment (start 193.04 104.4575) (end 195.10375 102.39375) (width 0.2) (layer "F.Cu") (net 1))
 (segment (start 216.69375 64.29375) (end 214.3125 61.9125) (width 0.2) (layer "F.Cu") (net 1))
 (via (at 209.55 102.39375) (size 0.6) (drill 0.3) (layers "F.Cu" "B.Cu") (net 1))
 (via (at 188.11875 61.9125) (size 0.6) (drill 0.3) (layers "F.Cu" "B.Cu") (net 1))
 (via (at 216.69375 95.25) (size 0.6) (drill 0.3) (layers "F.Cu" "B.Cu") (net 1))
 (segment (start 187.62 58.50125) (end 187.62 56.256) (width 0.2) (layer "B.Cu") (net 1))
 (segment (start 211.93125 102.39375) (end 216.69375 97.63125) (width 0.2) (layer "B.Cu") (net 1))
 (segment (start 188.11875 61.9125) (end 188.11875 59) (width 0.2) (layer "B.Cu") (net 1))
 (segment (start 216.69375 97.63125) (end 216.69375 95.25) (width 0.2) (layer "B.Cu") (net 1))
 (segment (start 209.55 102.39375) (end 211.93125 102.39375) (width 0.2) (layer "B.Cu") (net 1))
 (segment (start 188.11875 59) (end 187.62 58.50125) (width 0.2) (layer "B.Cu") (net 1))
 (segment (start 185.7375 59.53125) (end 198.46875 59.53125) (width 0.2) (layer "F.Cu") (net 15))
 (segment (start 198.46875 59.53125) (end 199 59) (width 0.2) (layer "F.Cu") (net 15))
 (segment (start 199 59) (end 199 57.576) (width 0.2) (layer "F.Cu") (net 15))
 (segment (start 199 57.576) (end 200.32 56.256) (width 0.2) (layer "F.Cu") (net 15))
 (via (at 185.7375 59.53125) (size 0.6) (drill 0.3) (layers "F.Cu" "B.Cu") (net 15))
 (segment (start 185.7375 59.53125) (end 183.35625 61.9125) (width 0.2) (layer "B.Cu") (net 15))
 (segment (start 164.30625 79.48525) (end 168.741 83.92) (width 0.2) (layer "B.Cu") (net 15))
 (segment (start 164.30625 61.9125) (end 164.30625 79.48525) (width 0.2) (layer "B.Cu") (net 15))
 (segment (start 183.35625 61.9125) (end 164.30625 61.9125) (width 0.2) (layer "B.Cu") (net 15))
 (segment (start 154.78125 38.1) (end 154.78125 64.29375) (width 0.2) (layer "F.Cu") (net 37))
 (segment (start 176.262 35.76825) (end 171.45 30.95625) (width 0.2) (layer "F.Cu") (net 37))
 (segment (start 176.262 38.476) (end 176.262 35.76825) (width 0.2) (layer "F.Cu") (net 37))
 (segment (start 171.45 30.95625) (end 161.925 30.95625) (width 0.2) (layer "F.Cu") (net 37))
 (segment (start 176.262 38.476) (end 177.46 38.476) (width 0.2) (layer "F.Cu") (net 37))
 (segment (start 161.925 30.95625) (end 154.78125 38.1) (width 0.2) (layer "F.Cu") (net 37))
 (segment (start 166.7875 76.3) (end 168.741 76.3) (width 0.2) (layer "F.Cu") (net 37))
 (segment (start 154.78125 64.29375) (end 166.7875 76.3) (width 0.2) (layer "F.Cu") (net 37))
 (segment (start 169.06875 64.29375) (end 200.70625 64.29375) (width 0.2) (layer "B.Cu") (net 16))
 (segment (start 203 56.396) (end 202.86 56.256) (width 0.2) (layer "B.Cu") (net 16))
 (segment (start 168.741 81.38) (end 166.6875 79.3265) (width 0.2) (layer "B.Cu") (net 16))
 (segment (start 166.6875 79.3265) (end 166.6875 66.675) (width 0.2) (layer "B.Cu") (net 16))
 (segment (start 203 62) (end 203 56.396) (width 0.2) (layer "B.Cu") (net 16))
 (segment (start 166.6875 66.675) (end 169.06875 64.29375) (width 0.2) (layer "B.Cu") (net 16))
 (segment (start 200.70625 64.29375) (end 203 62) (width 0.2) (layer "B.Cu") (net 16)))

